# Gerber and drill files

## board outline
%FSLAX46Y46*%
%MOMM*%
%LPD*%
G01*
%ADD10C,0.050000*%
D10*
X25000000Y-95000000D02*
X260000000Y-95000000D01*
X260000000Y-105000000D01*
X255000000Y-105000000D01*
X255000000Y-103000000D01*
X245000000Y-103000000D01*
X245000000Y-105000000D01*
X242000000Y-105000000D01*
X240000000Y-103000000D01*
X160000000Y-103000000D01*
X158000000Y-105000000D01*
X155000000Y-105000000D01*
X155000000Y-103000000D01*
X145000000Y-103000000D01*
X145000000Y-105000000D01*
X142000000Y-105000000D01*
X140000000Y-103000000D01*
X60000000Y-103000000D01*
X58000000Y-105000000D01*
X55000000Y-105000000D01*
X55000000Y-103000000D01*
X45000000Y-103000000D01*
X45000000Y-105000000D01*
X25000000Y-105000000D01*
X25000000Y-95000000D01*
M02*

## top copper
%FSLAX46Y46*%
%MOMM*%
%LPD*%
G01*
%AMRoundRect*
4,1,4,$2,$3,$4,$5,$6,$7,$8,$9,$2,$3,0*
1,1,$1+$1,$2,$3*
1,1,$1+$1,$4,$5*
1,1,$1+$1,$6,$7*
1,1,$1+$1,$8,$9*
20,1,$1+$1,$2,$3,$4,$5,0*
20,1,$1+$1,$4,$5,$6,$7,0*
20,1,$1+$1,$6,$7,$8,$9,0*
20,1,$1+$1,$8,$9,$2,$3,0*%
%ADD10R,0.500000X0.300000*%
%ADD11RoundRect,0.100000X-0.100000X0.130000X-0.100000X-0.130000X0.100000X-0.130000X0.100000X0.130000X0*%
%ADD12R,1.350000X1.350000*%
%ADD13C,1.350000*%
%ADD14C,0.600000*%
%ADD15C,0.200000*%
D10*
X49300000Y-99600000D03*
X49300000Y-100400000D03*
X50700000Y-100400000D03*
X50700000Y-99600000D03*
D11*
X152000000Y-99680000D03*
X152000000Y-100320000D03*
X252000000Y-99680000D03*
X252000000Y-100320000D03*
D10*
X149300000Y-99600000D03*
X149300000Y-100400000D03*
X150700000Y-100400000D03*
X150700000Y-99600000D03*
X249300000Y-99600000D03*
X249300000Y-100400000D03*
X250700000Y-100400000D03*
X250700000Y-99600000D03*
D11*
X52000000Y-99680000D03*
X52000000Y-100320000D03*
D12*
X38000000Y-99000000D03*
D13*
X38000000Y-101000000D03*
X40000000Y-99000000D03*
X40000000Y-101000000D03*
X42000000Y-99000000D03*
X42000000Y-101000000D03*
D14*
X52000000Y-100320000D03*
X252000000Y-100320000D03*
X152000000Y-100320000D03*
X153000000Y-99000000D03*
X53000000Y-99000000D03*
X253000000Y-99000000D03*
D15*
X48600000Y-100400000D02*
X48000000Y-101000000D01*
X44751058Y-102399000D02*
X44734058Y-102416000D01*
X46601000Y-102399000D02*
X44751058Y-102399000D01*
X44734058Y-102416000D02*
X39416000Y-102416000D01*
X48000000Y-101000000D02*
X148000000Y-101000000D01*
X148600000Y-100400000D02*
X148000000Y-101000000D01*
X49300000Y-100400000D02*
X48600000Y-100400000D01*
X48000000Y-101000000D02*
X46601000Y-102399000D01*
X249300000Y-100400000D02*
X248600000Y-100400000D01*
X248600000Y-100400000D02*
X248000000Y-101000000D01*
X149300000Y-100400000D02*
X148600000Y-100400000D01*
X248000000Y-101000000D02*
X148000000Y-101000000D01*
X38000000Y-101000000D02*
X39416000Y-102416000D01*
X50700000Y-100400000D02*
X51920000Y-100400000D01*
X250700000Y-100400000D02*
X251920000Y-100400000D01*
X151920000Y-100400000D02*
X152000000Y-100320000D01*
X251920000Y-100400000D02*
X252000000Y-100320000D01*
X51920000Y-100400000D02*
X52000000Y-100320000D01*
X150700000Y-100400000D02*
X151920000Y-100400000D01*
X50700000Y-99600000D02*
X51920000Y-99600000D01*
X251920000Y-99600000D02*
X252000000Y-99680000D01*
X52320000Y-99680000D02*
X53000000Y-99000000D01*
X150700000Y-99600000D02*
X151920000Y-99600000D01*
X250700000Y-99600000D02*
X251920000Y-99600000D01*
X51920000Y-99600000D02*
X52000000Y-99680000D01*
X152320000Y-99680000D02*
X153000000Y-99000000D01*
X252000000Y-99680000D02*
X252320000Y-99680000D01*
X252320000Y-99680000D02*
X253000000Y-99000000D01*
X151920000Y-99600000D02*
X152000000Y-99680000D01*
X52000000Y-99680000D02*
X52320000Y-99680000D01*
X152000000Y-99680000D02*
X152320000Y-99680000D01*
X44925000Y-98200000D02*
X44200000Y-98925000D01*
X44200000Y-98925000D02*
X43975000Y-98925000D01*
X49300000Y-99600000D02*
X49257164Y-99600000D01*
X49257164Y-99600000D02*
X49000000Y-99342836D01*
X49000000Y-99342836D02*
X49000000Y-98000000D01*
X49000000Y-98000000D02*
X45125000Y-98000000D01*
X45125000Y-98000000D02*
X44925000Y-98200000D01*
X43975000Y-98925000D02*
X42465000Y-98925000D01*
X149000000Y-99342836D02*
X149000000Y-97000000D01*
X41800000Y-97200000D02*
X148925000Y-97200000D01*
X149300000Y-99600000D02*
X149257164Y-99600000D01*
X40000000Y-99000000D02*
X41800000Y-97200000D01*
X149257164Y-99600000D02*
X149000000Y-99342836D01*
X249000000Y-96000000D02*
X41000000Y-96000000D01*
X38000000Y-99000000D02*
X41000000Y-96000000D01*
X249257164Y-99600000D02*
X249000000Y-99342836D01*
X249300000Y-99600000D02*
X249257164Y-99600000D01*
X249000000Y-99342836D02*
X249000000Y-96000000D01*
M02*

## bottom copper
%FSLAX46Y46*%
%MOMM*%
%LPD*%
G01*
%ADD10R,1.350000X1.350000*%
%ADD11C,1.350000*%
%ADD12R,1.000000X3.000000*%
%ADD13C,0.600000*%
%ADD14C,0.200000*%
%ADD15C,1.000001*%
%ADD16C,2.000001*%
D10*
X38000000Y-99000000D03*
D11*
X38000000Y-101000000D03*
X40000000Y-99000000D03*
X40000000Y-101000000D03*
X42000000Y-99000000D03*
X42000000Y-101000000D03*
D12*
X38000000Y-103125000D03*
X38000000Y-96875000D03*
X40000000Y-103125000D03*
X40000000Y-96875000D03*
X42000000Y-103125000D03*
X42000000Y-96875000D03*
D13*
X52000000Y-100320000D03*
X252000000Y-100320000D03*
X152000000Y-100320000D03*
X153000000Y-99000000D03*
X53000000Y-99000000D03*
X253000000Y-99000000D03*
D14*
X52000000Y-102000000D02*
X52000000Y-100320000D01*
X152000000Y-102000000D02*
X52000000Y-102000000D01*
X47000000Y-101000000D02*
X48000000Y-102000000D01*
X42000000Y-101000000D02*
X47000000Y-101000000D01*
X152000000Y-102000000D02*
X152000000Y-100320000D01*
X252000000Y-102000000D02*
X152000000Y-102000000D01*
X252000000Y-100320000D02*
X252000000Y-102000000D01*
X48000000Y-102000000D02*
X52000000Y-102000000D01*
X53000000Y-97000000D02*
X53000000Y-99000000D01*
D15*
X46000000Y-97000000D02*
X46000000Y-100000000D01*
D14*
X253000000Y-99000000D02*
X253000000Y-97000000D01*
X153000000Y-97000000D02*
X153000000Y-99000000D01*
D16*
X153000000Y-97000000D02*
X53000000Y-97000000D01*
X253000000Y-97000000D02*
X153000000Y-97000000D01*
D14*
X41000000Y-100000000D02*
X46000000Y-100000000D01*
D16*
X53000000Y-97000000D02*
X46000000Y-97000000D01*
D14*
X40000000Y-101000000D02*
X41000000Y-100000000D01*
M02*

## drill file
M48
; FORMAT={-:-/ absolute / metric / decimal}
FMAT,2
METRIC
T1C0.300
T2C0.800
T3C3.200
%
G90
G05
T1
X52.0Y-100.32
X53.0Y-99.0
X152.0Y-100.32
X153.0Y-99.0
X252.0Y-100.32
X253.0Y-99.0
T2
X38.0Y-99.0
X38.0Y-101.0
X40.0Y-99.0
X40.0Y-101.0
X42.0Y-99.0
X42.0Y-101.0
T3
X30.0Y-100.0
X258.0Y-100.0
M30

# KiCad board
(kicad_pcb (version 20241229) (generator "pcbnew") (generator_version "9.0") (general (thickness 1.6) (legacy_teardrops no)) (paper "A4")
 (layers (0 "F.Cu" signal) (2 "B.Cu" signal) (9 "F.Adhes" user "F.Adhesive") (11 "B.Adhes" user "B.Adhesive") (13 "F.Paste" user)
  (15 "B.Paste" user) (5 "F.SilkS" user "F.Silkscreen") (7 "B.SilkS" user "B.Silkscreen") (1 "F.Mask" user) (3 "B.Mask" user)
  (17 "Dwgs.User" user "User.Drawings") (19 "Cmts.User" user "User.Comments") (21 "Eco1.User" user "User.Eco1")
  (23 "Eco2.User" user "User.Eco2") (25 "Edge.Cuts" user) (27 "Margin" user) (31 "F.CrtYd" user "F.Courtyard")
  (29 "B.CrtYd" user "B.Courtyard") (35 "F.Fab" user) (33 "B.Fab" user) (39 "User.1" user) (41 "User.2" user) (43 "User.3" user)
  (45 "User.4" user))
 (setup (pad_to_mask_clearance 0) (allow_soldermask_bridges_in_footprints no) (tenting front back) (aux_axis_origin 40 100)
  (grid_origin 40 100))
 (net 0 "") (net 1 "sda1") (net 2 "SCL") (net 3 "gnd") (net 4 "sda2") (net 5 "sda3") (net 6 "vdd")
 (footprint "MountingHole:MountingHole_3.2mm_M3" (layer "F.Cu") (at 258 100)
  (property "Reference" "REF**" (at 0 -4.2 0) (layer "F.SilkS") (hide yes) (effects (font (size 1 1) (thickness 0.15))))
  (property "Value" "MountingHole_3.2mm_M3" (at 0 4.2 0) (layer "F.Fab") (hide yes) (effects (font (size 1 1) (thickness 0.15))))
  (pad "" np_thru_hole circle (at 0 0) (size 3.2 3.2) (drill 3.2) (layers "*.Cu" "*.Mask")))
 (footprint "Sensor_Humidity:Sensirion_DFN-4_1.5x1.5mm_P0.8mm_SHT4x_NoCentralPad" (layer "F.Cu") (at 50 100)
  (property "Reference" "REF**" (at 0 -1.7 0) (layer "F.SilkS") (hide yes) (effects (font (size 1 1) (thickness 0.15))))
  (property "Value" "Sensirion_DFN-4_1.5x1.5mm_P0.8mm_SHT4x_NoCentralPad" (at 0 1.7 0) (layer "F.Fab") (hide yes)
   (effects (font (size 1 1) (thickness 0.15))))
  (pad "1" smd rect (at -0.7 -0.4) (size 0.5 0.3) (layers "F.Cu" "F.Mask" "F.Paste") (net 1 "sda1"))
  (pad "2" smd rect (at -0.7 0.4) (size 0.5 0.3) (layers "F.Cu" "F.Mask" "F.Paste") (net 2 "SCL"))
  (pad "3" smd rect (at 0.7 0.4) (size 0.5 0.3) (layers "F.Cu" "F.Mask" "F.Paste"))
  (pad "4" smd rect (at 0.7 -0.4) (size 0.5 0.3) (layers "F.Cu" "F.Mask" "F.Paste") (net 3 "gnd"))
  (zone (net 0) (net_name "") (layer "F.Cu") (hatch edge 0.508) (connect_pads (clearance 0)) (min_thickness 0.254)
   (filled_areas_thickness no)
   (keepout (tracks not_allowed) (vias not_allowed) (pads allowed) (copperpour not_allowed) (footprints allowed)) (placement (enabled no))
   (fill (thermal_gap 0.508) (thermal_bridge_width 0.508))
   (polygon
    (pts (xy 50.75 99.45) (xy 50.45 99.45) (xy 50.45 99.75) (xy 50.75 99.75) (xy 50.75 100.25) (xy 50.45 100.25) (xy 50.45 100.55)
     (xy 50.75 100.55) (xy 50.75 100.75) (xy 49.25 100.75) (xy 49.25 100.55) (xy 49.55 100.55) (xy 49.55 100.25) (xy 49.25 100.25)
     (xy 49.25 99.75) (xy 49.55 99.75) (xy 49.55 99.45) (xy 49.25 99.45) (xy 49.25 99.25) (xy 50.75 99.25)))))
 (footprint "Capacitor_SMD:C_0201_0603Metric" (layer "F.Cu") (at 152 100 -90)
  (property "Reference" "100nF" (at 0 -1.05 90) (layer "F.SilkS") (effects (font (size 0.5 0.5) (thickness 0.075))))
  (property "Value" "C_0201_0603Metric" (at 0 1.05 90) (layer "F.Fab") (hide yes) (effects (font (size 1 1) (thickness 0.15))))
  (pad "" smd roundrect (at -0.345 0 270) (size 0.318 0.36) (layers "F.Paste") (roundrect_rratio 0.25))
  (pad "" smd roundrect (at 0.345 0 270) (size 0.318 0.36) (layers "F.Paste") (roundrect_rratio 0.25))
  (pad "1" smd roundrect (at -0.32 0 270) (size 0.46 0.4) (layers "F.Cu" "F.Mask") (roundrect_rratio 0.25))
  (pad "2" smd roundrect (at 0.32 0 270) (size 0.46 0.4) (layers "F.Cu" "F.Mask") (roundrect_rratio 0.25)))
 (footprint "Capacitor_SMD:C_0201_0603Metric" (layer "F.Cu") (at 252 100 -90)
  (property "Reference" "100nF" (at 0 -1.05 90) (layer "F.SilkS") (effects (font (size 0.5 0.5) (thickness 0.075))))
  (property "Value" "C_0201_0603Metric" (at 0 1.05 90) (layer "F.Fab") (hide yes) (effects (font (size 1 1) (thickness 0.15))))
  (pad "" smd roundrect (at -0.345 0 270) (size 0.318 0.36) (layers "F.Paste") (roundrect_rratio 0.25))
  (pad "" smd roundrect (at 0.345 0 270) (size 0.318 0.36) (layers "F.Paste") (roundrect_rratio 0.25))
  (pad "1" smd roundrect (at -0.32 0 270) (size 0.46 0.4) (layers "F.Cu" "F.Mask") (roundrect_rratio 0.25))
  (pad "2" smd roundrect (at 0.32 0 270) (size 0.46 0.4) (layers "F.Cu" "F.Mask") (roundrect_rratio 0.25)))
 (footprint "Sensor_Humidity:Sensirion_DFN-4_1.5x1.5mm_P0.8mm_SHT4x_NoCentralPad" (layer "F.Cu") (at 150 100)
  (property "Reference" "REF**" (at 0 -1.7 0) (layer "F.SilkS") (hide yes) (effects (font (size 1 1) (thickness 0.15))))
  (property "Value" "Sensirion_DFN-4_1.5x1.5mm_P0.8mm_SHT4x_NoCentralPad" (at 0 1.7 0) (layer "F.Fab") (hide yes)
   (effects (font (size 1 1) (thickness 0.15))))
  (pad "1" smd rect (at -0.7 -0.4) (size 0.5 0.3) (layers "F.Cu" "F.Mask" "F.Paste") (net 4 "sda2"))
  (pad "2" smd rect (at -0.7 0.4) (size 0.5 0.3) (layers "F.Cu" "F.Mask" "F.Paste") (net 2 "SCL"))
  (pad "3" smd rect (at 0.7 0.4) (size 0.5 0.3) (layers "F.Cu" "F.Mask" "F.Paste"))
  (pad "4" smd rect (at 0.7 -0.4) (size 0.5 0.3) (layers "F.Cu" "F.Mask" "F.Paste"))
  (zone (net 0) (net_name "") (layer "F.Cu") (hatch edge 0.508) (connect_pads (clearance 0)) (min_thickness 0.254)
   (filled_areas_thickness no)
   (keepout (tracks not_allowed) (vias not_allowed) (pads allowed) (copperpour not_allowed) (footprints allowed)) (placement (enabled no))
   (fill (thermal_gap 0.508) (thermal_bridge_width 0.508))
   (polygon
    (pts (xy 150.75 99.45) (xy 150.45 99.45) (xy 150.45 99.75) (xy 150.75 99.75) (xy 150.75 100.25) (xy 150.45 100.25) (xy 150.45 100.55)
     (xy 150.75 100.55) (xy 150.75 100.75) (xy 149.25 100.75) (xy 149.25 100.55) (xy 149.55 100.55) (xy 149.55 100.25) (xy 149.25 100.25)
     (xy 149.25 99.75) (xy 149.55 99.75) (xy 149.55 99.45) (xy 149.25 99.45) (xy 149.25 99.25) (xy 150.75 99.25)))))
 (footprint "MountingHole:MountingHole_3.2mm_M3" (layer "F.Cu") (at 30 100)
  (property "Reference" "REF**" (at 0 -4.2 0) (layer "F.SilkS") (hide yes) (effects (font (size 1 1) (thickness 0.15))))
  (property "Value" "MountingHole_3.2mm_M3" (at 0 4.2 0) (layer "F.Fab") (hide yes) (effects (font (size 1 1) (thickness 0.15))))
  (pad "" np_thru_hole circle (at 0 0) (size 3.2 3.2) (drill 3.2) (layers "*.Cu" "*.Mask")))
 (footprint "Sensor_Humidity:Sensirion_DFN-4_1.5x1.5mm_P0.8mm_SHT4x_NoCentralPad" (layer "F.Cu") (at 250 100)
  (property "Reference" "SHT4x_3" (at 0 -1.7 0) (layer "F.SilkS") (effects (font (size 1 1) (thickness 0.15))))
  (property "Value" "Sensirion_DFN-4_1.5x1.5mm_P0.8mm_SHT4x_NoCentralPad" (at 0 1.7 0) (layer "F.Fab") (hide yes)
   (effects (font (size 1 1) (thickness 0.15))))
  (pad "1" smd rect (at -0.7 -0.4) (size 0.5 0.3) (layers "F.Cu" "F.Mask" "F.Paste") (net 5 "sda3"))
  (pad "2" smd rect (at -0.7 0.4) (size 0.5 0.3) (layers "F.Cu" "F.Mask" "F.Paste") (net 2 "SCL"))
  (pad "3" smd rect (at 0.7 0.4) (size 0.5 0.3) (layers "F.Cu" "F.Mask" "F.Paste") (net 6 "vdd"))
  (pad "4" smd rect (at 0.7 -0.4) (size 0.5 0.3) (layers "F.Cu" "F.Mask" "F.Paste"))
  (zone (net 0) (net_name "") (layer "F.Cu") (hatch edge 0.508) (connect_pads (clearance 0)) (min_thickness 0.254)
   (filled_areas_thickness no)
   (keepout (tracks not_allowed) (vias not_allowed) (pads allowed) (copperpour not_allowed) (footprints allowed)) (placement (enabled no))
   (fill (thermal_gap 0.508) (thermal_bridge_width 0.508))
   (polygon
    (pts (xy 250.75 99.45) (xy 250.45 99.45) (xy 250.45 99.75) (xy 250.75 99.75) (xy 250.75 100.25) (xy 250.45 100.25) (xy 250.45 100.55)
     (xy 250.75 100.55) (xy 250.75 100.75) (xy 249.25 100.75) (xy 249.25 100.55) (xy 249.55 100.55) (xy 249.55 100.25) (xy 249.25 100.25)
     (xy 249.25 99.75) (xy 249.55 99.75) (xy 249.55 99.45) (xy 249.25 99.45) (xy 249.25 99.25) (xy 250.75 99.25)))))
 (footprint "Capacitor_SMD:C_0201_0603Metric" (layer "F.Cu") (at 52 100 -90)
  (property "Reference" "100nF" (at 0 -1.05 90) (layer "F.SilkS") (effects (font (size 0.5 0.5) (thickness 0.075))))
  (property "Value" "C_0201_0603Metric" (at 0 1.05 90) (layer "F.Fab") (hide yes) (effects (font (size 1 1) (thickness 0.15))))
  (pad "" smd roundrect (at -0.345 0 270) (size 0.318 0.36) (layers "F.Paste") (roundrect_rratio 0.25))
  (pad "" smd roundrect (at 0.345 0 270) (size 0.318 0.36) (layers "F.Paste") (roundrect_rratio 0.25))
  (pad "1" smd roundrect (at -0.32 0 270) (size 0.46 0.4) (layers "F.Cu" "F.Mask") (roundrect_rratio 0.25))
  (pad "2" smd roundrect (at 0.32 0 270) (size 0.46 0.4) (layers "F.Cu" "F.Mask") (roundrect_rratio 0.25)))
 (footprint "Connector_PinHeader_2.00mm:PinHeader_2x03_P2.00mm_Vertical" (layer "B.Cu") (at 38 99 -90)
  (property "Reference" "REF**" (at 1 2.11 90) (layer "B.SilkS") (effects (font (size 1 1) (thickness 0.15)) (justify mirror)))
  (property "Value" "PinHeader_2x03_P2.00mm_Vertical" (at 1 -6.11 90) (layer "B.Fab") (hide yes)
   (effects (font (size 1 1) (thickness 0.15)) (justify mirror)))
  (pad "1" thru_hole rect (at 0 0 270) (size 1.35 1.35) (drill 0.8) (layers "*.Cu" "*.Mask") (remove_unused_layers no) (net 5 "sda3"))
  (pad "2" thru_hole circle (at 2 0 270) (size 1.35 1.35) (drill 0.8) (layers "*.Cu" "*.Mask") (remove_unused_layers no) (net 2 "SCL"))
  (pad "3" thru_hole circle (at 0 -2 270) (size 1.35 1.35) (drill 0.8) (layers "*.Cu" "*.Mask") (remove_unused_layers no) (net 4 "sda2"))
  (pad "4" thru_hole circle (at 2 -2 270) (size 1.35 1.35) (drill 0.8) (layers "*.Cu" "*.Mask") (remove_unused_layers no) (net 3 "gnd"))
  (pad "5" thru_hole circle (at 0 -4 270) (size 1.35 1.35) (drill 0.8) (layers "*.Cu" "*.Mask") (remove_unused_layers no) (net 1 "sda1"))
  (pad "6" thru_hole circle (at 2 -4 270) (size 1.35 1.35) (drill 0.8) (layers "*.Cu" "*.Mask") (remove_unused_layers no) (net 6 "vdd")))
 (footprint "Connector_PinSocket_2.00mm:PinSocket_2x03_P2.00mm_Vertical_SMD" (layer "B.Cu") (at 40 100 -90)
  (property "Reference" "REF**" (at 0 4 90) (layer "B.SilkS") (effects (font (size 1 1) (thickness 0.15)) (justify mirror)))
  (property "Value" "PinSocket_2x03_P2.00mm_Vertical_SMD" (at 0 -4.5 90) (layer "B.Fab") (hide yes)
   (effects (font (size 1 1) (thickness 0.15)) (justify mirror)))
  (pad "1" smd rect (at 3.125 2 270) (size 3 1) (layers "B.Cu" "B.Mask" "B.Paste") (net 2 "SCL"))
  (pad "2" smd rect (at -3.125 2 270) (size 3 1) (layers "B.Cu" "B.Mask" "B.Paste") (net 5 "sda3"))
  (pad "3" smd rect (at 3.125 0 270) (size 3 1) (layers "B.Cu" "B.Mask" "B.Paste") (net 3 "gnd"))
  (pad "4" smd rect (at -3.125 0 270) (size 3 1) (layers "B.Cu" "B.Mask" "B.Paste") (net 4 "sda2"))
  (pad "5" smd rect (at 3.125 -2 270) (size 3 1) (layers "B.Cu" "B.Mask" "B.Paste") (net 6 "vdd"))
  (pad "6" smd rect (at -3.125 -2 270) (size 3 1) (layers "B.Cu" "B.Mask" "B.Paste") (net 1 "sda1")))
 (gr_poly
  (pts (xy 25 95) (xy 260 95) (xy 260 105) (xy 255 105) (xy 255 103) (xy 245 103) (xy 245 105) (xy 242 105) (xy 240 103) (xy 160 103)
   (xy 158 105) (xy 155 105) (xy 155 103) (xy 145 103) (xy 145 105) (xy 142 105) (xy 140 103) (xy 60 103) (xy 58 105) (xy 55 105)
   (xy 55 103) (xy 45 103) (xy 45 105) (xy 25 105))
  (stroke (width 0.05) (type solid)) (fill no) (layer "Edge.Cuts"))
 (segment (start 48.6 100.4) (end 48 101) (width 0.2) (layer "F.Cu") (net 2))
 (segment (start 44.751058 102.399) (end 44.734058 102.416) (width 0.2) (layer "F.Cu") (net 2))
 (segment (start 46.601 102.399) (end 44.751058 102.399) (width 0.2) (layer "F.Cu") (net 2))
 (segment (start 44.734058 102.416) (end 39.416 102.416) (width 0.2) (layer "F.Cu") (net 2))
 (segment (start 48 101) (end 148 101) (width 0.2) (layer "F.Cu") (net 2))
 (segment (start 148.6 100.4) (end 148 101) (width 0.2) (layer "F.Cu") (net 2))
 (segment (start 49.3 100.4) (end 48.6 100.4) (width 0.2) (layer "F.Cu") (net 2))
 (segment (start 48 101) (end 46.601 102.399) (width 0.2) (layer "F.Cu") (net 2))
 (segment (start 249.3 100.4) (end 248.6 100.4) (width 0.2) (layer "F.Cu") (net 2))
 (segment (start 248.6 100.4) (end 248 101) (width 0.2) (layer "F.Cu") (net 2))
 (segment (start 149.3 100.4) (end 148.6 100.4) (width 0.2) (layer "F.Cu") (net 2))
 (segment (start 248 101) (end 148 101) (width 0.2) (layer "F.Cu") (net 2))
 (segment (start 38 101) (end 39.416 102.416) (width 0.2) (layer "F.Cu") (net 2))
 (segment (start 50.7 100.4) (end 51.92 100.4) (width 0.2) (layer "F.Cu") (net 6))
 (segment (start 250.7 100.4) (end 251.92 100.4) (width 0.2) (layer "F.Cu") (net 6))
 (segment (start 151.92 100.4) (end 152 100.32) (width 0.2) (layer "F.Cu") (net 6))
 (segment (start 251.92 100.4) (end 252 100.32) (width 0.2) (layer "F.Cu") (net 6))
 (segment (start 51.92 100.4) (end 52 100.32) (width 0.2) (layer "F.Cu") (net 6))
 (segment (start 150.7 100.4) (end 151.92 100.4) (width 0.2) (layer "F.Cu") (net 6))
 (via blind (at 52 100.32) (size 0.6) (drill 0.3) (layers "F.Cu" "B.Cu") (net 6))
 (via blind (at 252 100.32) (size 0.6) (drill 0.3) (layers "F.Cu" "B.Cu") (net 6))
 (via blind (at 152 100.32) (size 0.6) (drill 0.3) (layers "F.Cu" "B.Cu") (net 6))
 (segment (start 52 102) (end 52 100.32) (width 0.2) (layer "B.Cu") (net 6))
 (segment (start 152 102) (end 52 102) (width 0.2) (layer "B.Cu") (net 6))
 (segment (start 47 101) (end 48 102) (width 0.2) (layer "B.Cu") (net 6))
 (segment (start 42 101) (end 47 101) (width 0.2) (layer "B.Cu") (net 6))
 (segment (start 152 102) (end 152 100.32) (width 0.2) (layer "B.Cu") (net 6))
 (segment (start 252 102) (end 152 102) (width 0.2) (layer "B.Cu") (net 6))
 (segment (start 252 100.32) (end 252 102) (width 0.2) (layer "B.Cu") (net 6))
 (segment (start 48 102) (end 52 102) (width 0.2) (layer "B.Cu") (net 6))
 (segment (start 50.7 99.6) (end 51.92 99.6) (width 0.2) (layer "F.Cu") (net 3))
 (segment (start 251.92 99.6) (end 252 99.68) (width 0.2) (layer "F.Cu") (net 3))
 (segment (start 52.32 99.68) (end 53 99) (width 0.2) (layer "F.Cu") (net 3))
 (segment (start 150.7 99.6) (end 151.92 99.6) (width 0.2) (layer "F.Cu") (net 3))
 (segment (start 250.7 99.6) (end 251.92 99.6) (width 0.2) (layer "F.Cu") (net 3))
 (segment (start 51.92 99.6) (end 52 99.68) (width 0.2) (layer "F.Cu") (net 3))
 (segment (start 152.32 99.68) (end 153 99) (width 0.2) (layer "F.Cu") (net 3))
 (segment (start 252 99.68) (end 252.32 99.68) (width 0.2) (layer "F.Cu") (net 3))
 (segment (start 252.32 99.68) (end 253 99) (width 0.2) (layer "F.Cu") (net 3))
 (segment (start 151.92 99.6) (end 152 99.68) (width 0.2) (layer "F.Cu") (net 3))
 (segment (start 52 99.68) (end 52.32 99.68) (width 0.2) (layer "F.Cu") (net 3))
 (segment (start 152 99.68) (end 152.32 99.68) (width 0.2) (layer "F.Cu") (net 3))
 (via blind (at 153 99) (size 0.6) (drill 0.3) (layers "F.Cu" "B.Cu") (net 3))
 (via blind (at 53 99) (size 0.6) (drill 0.3) (layers "F.Cu" "B.Cu") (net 3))
 (via blind (at 253 99) (size 0.6) (drill 0.3) (layers "F.Cu" "B.Cu") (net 3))
 (segment (start 53 97) (end 53 99) (width 0.2) (layer "B.Cu") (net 3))
 (segment (start 46 97) (end 46 100) (width 1.000001) (layer "B.Cu") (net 3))
 (segment (start 253 99) (end 253 97) (width 0.2) (layer "B.Cu") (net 3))
 (segment (start 153 97) (end 153 99) (width 0.2) (layer "B.Cu") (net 3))
 (segment (start 153 97) (end 53 97) (width 2.000001) (layer "B.Cu") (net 3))
 (segment (start 253 97) (end 153 97) (width 2.000001) (layer "B.Cu") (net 3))
 (segment (start 41 100) (end 46 100) (width 0.2) (layer "B.Cu") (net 3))
 (segment (start 53 97) (end 46 97) (width 2.000001) (layer "B.Cu") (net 3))
 (segment (start 40 101) (end 41 100) (width 0.2) (layer "B.Cu") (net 3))
 (segment (start 44.925 98.2) (end 44.2 98.925) (width 0.2) (layer "F.Cu") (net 1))
 (segment (start 44.2 98.925) (end 43.975 98.925) (width 0.2) (layer "F.Cu") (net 1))
 (segment (start 49.3 99.6) (end 49.257164 99.6) (width 0.2) (layer "F.Cu") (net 1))
 (segment (start 49.257164 99.6) (end 49 99.342836) (width 0.2) (layer "F.Cu") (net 1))
 (segment (start 49 99.342836) (end 49 98) (width 0.2) (layer "F.Cu") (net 1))
 (segment (start 49 98) (end 45.125 98) (width 0.2) (layer "F.Cu") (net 1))
 (segment (start 45.125 98) (end 44.925 98.2) (width 0.2) (layer "F.Cu") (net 1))
 (segment (start 43.975 98.925) (end 42.465 98.925) (width 0.2) (layer "F.Cu") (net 1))
 (segment (start 149 99.342836) (end 149 97) (width 0.2) (layer "F.Cu") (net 4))
 (segment (start 41.8 97.2) (end 148.925 97.2) (width 0.2) (layer "F.Cu") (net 4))
 (segment (start 149.3 99.6) (end 149.257164 99.6) (width 0.2) (layer "F.Cu") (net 4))
 (segment (start 40 99) (end 41.8 97.2) (width 0.2) (layer "F.Cu") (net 4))
 (segment (start 149.257164 99.6) (end 149 99.342836) (width 0.2) (layer "F.Cu") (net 4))
 (segment (start 249 96) (end 41 96) (width 0.2) (layer "F.Cu") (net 5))
 (segment (start 38 99) (end 41 96) (width 0.2) (layer "F.Cu") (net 5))
 (segment (start 249.257164 99.6) (end 249 99.342836) (width 0.2) (layer "F.Cu") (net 5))
 (segment (start 249.3 99.6) (end 249.257164 99.6) (width 0.2) (layer "F.Cu") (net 5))
 (segment (start 249 99.342836) (end 249 96) (width 0.2) (layer "F.Cu") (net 5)))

